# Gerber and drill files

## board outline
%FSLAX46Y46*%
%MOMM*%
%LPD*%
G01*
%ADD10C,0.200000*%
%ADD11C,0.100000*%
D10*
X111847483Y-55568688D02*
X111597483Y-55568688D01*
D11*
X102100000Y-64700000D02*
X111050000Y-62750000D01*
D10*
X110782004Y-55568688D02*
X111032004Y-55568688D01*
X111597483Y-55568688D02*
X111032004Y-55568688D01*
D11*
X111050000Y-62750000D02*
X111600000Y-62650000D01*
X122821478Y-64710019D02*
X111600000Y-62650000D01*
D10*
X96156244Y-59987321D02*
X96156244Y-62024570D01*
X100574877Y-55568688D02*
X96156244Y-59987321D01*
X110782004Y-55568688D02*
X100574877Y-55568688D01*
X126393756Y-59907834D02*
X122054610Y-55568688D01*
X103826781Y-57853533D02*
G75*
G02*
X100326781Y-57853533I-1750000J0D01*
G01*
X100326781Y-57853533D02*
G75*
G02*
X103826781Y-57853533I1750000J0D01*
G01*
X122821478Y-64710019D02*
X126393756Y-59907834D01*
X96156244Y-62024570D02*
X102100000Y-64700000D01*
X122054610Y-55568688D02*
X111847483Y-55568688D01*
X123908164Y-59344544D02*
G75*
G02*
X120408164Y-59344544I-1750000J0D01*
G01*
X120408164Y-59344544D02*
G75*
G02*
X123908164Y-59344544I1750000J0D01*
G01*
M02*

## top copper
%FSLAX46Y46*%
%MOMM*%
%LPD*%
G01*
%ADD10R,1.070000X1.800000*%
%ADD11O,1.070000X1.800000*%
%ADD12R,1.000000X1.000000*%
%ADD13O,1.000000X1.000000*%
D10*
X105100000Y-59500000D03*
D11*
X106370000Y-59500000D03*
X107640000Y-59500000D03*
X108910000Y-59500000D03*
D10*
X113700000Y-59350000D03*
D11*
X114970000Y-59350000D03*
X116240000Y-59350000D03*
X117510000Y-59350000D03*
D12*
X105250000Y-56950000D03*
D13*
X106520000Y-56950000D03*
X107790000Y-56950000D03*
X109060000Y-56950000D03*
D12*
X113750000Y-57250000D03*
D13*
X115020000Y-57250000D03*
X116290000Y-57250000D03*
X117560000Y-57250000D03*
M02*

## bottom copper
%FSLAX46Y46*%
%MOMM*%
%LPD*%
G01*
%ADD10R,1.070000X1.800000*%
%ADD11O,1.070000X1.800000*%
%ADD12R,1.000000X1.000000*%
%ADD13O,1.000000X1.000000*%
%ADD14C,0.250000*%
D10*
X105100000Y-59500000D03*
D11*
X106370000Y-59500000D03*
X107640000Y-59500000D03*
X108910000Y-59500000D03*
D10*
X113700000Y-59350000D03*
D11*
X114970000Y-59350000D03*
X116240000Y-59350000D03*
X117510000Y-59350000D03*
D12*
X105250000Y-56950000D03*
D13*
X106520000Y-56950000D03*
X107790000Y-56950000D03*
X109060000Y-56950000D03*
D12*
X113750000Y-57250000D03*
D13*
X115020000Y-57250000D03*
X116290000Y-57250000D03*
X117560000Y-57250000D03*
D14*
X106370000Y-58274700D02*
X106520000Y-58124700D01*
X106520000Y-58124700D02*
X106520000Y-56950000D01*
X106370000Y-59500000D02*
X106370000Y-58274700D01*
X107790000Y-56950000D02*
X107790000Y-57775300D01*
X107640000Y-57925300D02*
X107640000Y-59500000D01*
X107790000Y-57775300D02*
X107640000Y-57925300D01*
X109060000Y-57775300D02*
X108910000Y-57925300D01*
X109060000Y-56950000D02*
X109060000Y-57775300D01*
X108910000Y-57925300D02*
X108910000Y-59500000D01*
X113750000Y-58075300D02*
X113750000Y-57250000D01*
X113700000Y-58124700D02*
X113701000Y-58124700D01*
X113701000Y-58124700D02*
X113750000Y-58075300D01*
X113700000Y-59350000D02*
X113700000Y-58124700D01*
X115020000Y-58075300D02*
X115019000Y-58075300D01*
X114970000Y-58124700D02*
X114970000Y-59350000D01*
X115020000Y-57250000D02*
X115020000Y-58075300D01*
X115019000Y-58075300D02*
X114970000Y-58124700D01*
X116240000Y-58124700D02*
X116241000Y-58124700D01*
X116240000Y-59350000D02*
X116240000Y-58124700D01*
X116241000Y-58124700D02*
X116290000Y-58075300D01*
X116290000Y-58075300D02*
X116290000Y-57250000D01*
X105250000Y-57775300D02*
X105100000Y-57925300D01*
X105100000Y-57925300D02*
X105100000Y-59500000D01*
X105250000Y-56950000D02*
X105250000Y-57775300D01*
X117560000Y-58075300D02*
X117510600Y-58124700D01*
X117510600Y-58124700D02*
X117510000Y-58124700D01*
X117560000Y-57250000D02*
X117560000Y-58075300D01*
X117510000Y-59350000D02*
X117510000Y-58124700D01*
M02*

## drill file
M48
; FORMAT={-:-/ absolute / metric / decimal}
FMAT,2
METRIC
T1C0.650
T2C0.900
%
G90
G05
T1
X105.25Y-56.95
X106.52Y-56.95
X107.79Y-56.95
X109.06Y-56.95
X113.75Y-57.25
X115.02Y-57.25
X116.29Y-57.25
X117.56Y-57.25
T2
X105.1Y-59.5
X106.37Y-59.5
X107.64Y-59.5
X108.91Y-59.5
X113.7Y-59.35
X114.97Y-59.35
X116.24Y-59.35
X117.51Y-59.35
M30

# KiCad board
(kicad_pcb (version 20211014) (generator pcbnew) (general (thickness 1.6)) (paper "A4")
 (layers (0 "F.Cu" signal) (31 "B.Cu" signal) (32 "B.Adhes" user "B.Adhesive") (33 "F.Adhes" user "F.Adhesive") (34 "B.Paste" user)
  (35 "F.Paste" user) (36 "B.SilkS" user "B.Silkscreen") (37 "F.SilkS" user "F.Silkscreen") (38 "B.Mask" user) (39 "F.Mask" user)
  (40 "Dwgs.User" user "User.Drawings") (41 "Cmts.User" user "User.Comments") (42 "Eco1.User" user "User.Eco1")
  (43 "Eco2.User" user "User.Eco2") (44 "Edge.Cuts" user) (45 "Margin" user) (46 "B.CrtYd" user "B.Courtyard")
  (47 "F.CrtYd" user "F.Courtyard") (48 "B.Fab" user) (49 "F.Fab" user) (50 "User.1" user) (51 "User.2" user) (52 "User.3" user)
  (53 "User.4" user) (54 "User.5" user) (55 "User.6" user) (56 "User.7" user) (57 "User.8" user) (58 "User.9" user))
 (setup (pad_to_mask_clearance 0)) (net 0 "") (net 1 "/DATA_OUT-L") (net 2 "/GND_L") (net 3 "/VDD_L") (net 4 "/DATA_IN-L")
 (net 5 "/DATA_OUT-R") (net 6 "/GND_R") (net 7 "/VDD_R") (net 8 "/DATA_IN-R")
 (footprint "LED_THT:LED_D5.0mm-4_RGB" (layer "F.Cu") (at 105.1 59.5)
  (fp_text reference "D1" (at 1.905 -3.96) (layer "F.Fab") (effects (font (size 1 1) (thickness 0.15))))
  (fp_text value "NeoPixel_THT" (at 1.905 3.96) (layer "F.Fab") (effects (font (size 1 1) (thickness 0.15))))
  (pad "1" thru_hole rect (at 0 0) (size 1.07 1.8) (drill 0.9) (layers *.Cu *.Mask) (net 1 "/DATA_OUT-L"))
  (pad "2" thru_hole oval (at 1.27 0) (size 1.07 1.8) (drill 0.9) (layers *.Cu *.Mask) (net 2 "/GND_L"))
  (pad "3" thru_hole oval (at 2.54 0) (size 1.07 1.8) (drill 0.9) (layers *.Cu *.Mask) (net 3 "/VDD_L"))
  (pad "4" thru_hole oval (at 3.81 0) (size 1.07 1.8) (drill 0.9) (layers *.Cu *.Mask) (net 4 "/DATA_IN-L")))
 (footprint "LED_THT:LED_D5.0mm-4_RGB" (layer "F.Cu") (at 113.7 59.35)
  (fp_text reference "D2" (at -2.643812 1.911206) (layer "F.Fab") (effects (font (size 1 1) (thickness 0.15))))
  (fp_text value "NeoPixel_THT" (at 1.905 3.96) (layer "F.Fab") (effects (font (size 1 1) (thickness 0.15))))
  (pad "1" thru_hole rect (at 0 0) (size 1.07 1.8) (drill 0.9) (layers *.Cu *.Mask) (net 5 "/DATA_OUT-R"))
  (pad "2" thru_hole oval (at 1.27 0) (size 1.07 1.8) (drill 0.9) (layers *.Cu *.Mask) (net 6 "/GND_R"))
  (pad "3" thru_hole oval (at 2.54 0) (size 1.07 1.8) (drill 0.9) (layers *.Cu *.Mask) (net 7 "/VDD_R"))
  (pad "4" thru_hole oval (at 3.81 0) (size 1.07 1.8) (drill 0.9) (layers *.Cu *.Mask) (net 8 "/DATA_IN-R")))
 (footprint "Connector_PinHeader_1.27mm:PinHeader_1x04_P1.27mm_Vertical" (layer "B.Cu") (at 105.25 56.95 -90)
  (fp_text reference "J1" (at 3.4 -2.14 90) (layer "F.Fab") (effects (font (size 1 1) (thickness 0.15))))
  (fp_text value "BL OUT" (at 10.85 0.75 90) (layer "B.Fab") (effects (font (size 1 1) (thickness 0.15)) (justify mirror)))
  (pad "1" thru_hole rect (at 0 0 270) (size 1 1) (drill 0.65) (layers *.Cu *.Mask) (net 1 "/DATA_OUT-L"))
  (pad "2" thru_hole oval (at 0 -1.27 270) (size 1 1) (drill 0.65) (layers *.Cu *.Mask) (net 2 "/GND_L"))
  (pad "3" thru_hole oval (at 0 -2.54 270) (size 1 1) (drill 0.65) (layers *.Cu *.Mask) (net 3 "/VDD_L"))
  (pad "4" thru_hole oval (at 0 -3.81 270) (size 1 1) (drill 0.65) (layers *.Cu *.Mask) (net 4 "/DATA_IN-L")))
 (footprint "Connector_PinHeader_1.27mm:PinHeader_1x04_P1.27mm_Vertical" (layer "B.Cu") (at 113.75 57.25 -90)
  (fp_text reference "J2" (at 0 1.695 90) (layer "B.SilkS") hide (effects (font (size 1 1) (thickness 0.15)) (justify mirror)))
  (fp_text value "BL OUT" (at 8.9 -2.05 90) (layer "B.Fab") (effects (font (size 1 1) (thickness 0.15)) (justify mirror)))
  (pad "1" thru_hole rect (at 0 0 270) (size 1 1) (drill 0.65) (layers *.Cu *.Mask) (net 5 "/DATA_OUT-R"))
  (pad "2" thru_hole oval (at 0 -1.27 270) (size 1 1) (drill 0.65) (layers *.Cu *.Mask) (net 6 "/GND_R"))
  (pad "3" thru_hole oval (at 0 -2.54 270) (size 1 1) (drill 0.65) (layers *.Cu *.Mask) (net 7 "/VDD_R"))
  (pad "4" thru_hole oval (at 0 -3.81 270) (size 1 1) (drill 0.65) (layers *.Cu *.Mask) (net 8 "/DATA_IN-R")))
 (gr_line (start 111.847483 55.568688) (end 111.597483 55.568688) (layer "Edge.Cuts") (width 0.2))
 (gr_line (start 102.1 64.7) (end 111.05 62.75) (layer "Edge.Cuts") (width 0.1))
 (gr_line (start 110.782004 55.568688) (end 111.032004 55.568688) (layer "Edge.Cuts") (width 0.2))
 (gr_line (start 111.597483 55.568688) (end 111.032004 55.568688) (layer "Edge.Cuts") (width 0.2))
 (gr_line (start 111.05 62.75) (end 111.6 62.65) (layer "Edge.Cuts") (width 0.1))
 (gr_line (start 122.821478 64.710019) (end 111.6 62.65) (layer "Edge.Cuts") (width 0.1))
 (gr_line (start 96.156244 59.987321) (end 96.156244 62.02457) (layer "Edge.Cuts") (width 0.2))
 (gr_line (start 100.574877 55.568688) (end 96.156244 59.987321) (layer "Edge.Cuts") (width 0.2))
 (gr_line (start 110.782004 55.568688) (end 100.574877 55.568688) (layer "Edge.Cuts") (width 0.2))
 (gr_line (start 126.393756 59.907834) (end 122.05461 55.568688) (layer "Edge.Cuts") (width 0.2))
 (gr_circle (center 102.076781 57.853533) (end 103.826781 57.853533) (layer "Edge.Cuts") (width 0.2) (fill none))
 (gr_line (start 122.821478 64.710019) (end 126.393756 59.907834) (layer "Edge.Cuts") (width 0.2))
 (gr_line (start 96.156244 62.02457) (end 102.1 64.7) (layer "Edge.Cuts") (width 0.2))
 (gr_line (start 122.05461 55.568688) (end 111.847483 55.568688) (layer "Edge.Cuts") (width 0.2))
 (gr_circle (center 122.158164 59.344544) (end 123.908164 59.344544) (layer "Edge.Cuts") (width 0.2) (fill none))
 (segment (start 106.37 58.2747) (end 106.52 58.1247) (width 0.25) (layer "B.Cu") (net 2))
 (segment (start 106.52 58.1247) (end 106.52 56.95) (width 0.25) (layer "B.Cu") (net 2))
 (segment (start 106.37 59.5) (end 106.37 58.2747) (width 0.25) (layer "B.Cu") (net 2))
 (segment (start 107.79 56.95) (end 107.79 57.7753) (width 0.25) (layer "B.Cu") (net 3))
 (segment (start 107.64 57.9253) (end 107.64 59.5) (width 0.25) (layer "B.Cu") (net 3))
 (segment (start 107.79 57.7753) (end 107.64 57.9253) (width 0.25) (layer "B.Cu") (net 3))
 (segment (start 109.06 57.7753) (end 108.91 57.9253) (width 0.25) (layer "B.Cu") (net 4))
 (segment (start 109.06 56.95) (end 109.06 57.7753) (width 0.25) (layer "B.Cu") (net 4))
 (segment (start 108.91 57.9253) (end 108.91 59.5) (width 0.25) (layer "B.Cu") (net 4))
 (segment (start 113.75 58.0753) (end 113.75 57.25) (width 0.25) (layer "B.Cu") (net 5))
 (segment (start 113.7 58.1247) (end 113.701 58.1247) (width 0.25) (layer "B.Cu") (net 5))
 (segment (start 113.701 58.1247) (end 113.75 58.0753) (width 0.25) (layer "B.Cu") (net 5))
 (segment (start 113.7 59.35) (end 113.7 58.1247) (width 0.25) (layer "B.Cu") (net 5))
 (segment (start 115.02 58.0753) (end 115.019 58.0753) (width 0.25) (layer "B.Cu") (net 6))
 (segment (start 114.97 58.1247) (end 114.97 59.35) (width 0.25) (layer "B.Cu") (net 6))
 (segment (start 115.02 57.25) (end 115.02 58.0753) (width 0.25) (layer "B.Cu") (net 6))
 (segment (start 115.019 58.0753) (end 114.97 58.1247) (width 0.25) (layer "B.Cu") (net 6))
 (segment (start 116.24 58.1247) (end 116.241 58.1247) (width 0.25) (layer "B.Cu") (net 7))
 (segment (start 116.24 59.35) (end 116.24 58.1247) (width 0.25) (layer "B.Cu") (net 7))
 (segment (start 116.241 58.1247) (end 116.29 58.0753) (width 0.25) (layer "B.Cu") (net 7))
 (segment (start 116.29 58.0753) (end 116.29 57.25) (width 0.25) (layer "B.Cu") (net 7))
 (segment (start 105.25 57.7753) (end 105.1 57.9253) (width 0.25) (layer "B.Cu") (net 1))
 (segment (start 105.1 57.9253) (end 105.1 59.5) (width 0.25) (layer "B.Cu") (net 1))
 (segment (start 105.25 56.95) (end 105.25 57.7753) (width 0.25) (layer "B.Cu") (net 1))
 (segment (start 117.56 58.0753) (end 117.5106 58.1247) (width 0.25) (layer "B.Cu") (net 8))
 (segment (start 117.5106 58.1247) (end 117.51 58.1247) (width 0.25) (layer "B.Cu") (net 8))
 (segment (start 117.56 57.25) (end 117.56 58.0753) (width 0.25) (layer "B.Cu") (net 8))
 (segment (start 117.51 59.35) (end 117.51 58.1247) (width 0.25) (layer "B.Cu") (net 8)))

